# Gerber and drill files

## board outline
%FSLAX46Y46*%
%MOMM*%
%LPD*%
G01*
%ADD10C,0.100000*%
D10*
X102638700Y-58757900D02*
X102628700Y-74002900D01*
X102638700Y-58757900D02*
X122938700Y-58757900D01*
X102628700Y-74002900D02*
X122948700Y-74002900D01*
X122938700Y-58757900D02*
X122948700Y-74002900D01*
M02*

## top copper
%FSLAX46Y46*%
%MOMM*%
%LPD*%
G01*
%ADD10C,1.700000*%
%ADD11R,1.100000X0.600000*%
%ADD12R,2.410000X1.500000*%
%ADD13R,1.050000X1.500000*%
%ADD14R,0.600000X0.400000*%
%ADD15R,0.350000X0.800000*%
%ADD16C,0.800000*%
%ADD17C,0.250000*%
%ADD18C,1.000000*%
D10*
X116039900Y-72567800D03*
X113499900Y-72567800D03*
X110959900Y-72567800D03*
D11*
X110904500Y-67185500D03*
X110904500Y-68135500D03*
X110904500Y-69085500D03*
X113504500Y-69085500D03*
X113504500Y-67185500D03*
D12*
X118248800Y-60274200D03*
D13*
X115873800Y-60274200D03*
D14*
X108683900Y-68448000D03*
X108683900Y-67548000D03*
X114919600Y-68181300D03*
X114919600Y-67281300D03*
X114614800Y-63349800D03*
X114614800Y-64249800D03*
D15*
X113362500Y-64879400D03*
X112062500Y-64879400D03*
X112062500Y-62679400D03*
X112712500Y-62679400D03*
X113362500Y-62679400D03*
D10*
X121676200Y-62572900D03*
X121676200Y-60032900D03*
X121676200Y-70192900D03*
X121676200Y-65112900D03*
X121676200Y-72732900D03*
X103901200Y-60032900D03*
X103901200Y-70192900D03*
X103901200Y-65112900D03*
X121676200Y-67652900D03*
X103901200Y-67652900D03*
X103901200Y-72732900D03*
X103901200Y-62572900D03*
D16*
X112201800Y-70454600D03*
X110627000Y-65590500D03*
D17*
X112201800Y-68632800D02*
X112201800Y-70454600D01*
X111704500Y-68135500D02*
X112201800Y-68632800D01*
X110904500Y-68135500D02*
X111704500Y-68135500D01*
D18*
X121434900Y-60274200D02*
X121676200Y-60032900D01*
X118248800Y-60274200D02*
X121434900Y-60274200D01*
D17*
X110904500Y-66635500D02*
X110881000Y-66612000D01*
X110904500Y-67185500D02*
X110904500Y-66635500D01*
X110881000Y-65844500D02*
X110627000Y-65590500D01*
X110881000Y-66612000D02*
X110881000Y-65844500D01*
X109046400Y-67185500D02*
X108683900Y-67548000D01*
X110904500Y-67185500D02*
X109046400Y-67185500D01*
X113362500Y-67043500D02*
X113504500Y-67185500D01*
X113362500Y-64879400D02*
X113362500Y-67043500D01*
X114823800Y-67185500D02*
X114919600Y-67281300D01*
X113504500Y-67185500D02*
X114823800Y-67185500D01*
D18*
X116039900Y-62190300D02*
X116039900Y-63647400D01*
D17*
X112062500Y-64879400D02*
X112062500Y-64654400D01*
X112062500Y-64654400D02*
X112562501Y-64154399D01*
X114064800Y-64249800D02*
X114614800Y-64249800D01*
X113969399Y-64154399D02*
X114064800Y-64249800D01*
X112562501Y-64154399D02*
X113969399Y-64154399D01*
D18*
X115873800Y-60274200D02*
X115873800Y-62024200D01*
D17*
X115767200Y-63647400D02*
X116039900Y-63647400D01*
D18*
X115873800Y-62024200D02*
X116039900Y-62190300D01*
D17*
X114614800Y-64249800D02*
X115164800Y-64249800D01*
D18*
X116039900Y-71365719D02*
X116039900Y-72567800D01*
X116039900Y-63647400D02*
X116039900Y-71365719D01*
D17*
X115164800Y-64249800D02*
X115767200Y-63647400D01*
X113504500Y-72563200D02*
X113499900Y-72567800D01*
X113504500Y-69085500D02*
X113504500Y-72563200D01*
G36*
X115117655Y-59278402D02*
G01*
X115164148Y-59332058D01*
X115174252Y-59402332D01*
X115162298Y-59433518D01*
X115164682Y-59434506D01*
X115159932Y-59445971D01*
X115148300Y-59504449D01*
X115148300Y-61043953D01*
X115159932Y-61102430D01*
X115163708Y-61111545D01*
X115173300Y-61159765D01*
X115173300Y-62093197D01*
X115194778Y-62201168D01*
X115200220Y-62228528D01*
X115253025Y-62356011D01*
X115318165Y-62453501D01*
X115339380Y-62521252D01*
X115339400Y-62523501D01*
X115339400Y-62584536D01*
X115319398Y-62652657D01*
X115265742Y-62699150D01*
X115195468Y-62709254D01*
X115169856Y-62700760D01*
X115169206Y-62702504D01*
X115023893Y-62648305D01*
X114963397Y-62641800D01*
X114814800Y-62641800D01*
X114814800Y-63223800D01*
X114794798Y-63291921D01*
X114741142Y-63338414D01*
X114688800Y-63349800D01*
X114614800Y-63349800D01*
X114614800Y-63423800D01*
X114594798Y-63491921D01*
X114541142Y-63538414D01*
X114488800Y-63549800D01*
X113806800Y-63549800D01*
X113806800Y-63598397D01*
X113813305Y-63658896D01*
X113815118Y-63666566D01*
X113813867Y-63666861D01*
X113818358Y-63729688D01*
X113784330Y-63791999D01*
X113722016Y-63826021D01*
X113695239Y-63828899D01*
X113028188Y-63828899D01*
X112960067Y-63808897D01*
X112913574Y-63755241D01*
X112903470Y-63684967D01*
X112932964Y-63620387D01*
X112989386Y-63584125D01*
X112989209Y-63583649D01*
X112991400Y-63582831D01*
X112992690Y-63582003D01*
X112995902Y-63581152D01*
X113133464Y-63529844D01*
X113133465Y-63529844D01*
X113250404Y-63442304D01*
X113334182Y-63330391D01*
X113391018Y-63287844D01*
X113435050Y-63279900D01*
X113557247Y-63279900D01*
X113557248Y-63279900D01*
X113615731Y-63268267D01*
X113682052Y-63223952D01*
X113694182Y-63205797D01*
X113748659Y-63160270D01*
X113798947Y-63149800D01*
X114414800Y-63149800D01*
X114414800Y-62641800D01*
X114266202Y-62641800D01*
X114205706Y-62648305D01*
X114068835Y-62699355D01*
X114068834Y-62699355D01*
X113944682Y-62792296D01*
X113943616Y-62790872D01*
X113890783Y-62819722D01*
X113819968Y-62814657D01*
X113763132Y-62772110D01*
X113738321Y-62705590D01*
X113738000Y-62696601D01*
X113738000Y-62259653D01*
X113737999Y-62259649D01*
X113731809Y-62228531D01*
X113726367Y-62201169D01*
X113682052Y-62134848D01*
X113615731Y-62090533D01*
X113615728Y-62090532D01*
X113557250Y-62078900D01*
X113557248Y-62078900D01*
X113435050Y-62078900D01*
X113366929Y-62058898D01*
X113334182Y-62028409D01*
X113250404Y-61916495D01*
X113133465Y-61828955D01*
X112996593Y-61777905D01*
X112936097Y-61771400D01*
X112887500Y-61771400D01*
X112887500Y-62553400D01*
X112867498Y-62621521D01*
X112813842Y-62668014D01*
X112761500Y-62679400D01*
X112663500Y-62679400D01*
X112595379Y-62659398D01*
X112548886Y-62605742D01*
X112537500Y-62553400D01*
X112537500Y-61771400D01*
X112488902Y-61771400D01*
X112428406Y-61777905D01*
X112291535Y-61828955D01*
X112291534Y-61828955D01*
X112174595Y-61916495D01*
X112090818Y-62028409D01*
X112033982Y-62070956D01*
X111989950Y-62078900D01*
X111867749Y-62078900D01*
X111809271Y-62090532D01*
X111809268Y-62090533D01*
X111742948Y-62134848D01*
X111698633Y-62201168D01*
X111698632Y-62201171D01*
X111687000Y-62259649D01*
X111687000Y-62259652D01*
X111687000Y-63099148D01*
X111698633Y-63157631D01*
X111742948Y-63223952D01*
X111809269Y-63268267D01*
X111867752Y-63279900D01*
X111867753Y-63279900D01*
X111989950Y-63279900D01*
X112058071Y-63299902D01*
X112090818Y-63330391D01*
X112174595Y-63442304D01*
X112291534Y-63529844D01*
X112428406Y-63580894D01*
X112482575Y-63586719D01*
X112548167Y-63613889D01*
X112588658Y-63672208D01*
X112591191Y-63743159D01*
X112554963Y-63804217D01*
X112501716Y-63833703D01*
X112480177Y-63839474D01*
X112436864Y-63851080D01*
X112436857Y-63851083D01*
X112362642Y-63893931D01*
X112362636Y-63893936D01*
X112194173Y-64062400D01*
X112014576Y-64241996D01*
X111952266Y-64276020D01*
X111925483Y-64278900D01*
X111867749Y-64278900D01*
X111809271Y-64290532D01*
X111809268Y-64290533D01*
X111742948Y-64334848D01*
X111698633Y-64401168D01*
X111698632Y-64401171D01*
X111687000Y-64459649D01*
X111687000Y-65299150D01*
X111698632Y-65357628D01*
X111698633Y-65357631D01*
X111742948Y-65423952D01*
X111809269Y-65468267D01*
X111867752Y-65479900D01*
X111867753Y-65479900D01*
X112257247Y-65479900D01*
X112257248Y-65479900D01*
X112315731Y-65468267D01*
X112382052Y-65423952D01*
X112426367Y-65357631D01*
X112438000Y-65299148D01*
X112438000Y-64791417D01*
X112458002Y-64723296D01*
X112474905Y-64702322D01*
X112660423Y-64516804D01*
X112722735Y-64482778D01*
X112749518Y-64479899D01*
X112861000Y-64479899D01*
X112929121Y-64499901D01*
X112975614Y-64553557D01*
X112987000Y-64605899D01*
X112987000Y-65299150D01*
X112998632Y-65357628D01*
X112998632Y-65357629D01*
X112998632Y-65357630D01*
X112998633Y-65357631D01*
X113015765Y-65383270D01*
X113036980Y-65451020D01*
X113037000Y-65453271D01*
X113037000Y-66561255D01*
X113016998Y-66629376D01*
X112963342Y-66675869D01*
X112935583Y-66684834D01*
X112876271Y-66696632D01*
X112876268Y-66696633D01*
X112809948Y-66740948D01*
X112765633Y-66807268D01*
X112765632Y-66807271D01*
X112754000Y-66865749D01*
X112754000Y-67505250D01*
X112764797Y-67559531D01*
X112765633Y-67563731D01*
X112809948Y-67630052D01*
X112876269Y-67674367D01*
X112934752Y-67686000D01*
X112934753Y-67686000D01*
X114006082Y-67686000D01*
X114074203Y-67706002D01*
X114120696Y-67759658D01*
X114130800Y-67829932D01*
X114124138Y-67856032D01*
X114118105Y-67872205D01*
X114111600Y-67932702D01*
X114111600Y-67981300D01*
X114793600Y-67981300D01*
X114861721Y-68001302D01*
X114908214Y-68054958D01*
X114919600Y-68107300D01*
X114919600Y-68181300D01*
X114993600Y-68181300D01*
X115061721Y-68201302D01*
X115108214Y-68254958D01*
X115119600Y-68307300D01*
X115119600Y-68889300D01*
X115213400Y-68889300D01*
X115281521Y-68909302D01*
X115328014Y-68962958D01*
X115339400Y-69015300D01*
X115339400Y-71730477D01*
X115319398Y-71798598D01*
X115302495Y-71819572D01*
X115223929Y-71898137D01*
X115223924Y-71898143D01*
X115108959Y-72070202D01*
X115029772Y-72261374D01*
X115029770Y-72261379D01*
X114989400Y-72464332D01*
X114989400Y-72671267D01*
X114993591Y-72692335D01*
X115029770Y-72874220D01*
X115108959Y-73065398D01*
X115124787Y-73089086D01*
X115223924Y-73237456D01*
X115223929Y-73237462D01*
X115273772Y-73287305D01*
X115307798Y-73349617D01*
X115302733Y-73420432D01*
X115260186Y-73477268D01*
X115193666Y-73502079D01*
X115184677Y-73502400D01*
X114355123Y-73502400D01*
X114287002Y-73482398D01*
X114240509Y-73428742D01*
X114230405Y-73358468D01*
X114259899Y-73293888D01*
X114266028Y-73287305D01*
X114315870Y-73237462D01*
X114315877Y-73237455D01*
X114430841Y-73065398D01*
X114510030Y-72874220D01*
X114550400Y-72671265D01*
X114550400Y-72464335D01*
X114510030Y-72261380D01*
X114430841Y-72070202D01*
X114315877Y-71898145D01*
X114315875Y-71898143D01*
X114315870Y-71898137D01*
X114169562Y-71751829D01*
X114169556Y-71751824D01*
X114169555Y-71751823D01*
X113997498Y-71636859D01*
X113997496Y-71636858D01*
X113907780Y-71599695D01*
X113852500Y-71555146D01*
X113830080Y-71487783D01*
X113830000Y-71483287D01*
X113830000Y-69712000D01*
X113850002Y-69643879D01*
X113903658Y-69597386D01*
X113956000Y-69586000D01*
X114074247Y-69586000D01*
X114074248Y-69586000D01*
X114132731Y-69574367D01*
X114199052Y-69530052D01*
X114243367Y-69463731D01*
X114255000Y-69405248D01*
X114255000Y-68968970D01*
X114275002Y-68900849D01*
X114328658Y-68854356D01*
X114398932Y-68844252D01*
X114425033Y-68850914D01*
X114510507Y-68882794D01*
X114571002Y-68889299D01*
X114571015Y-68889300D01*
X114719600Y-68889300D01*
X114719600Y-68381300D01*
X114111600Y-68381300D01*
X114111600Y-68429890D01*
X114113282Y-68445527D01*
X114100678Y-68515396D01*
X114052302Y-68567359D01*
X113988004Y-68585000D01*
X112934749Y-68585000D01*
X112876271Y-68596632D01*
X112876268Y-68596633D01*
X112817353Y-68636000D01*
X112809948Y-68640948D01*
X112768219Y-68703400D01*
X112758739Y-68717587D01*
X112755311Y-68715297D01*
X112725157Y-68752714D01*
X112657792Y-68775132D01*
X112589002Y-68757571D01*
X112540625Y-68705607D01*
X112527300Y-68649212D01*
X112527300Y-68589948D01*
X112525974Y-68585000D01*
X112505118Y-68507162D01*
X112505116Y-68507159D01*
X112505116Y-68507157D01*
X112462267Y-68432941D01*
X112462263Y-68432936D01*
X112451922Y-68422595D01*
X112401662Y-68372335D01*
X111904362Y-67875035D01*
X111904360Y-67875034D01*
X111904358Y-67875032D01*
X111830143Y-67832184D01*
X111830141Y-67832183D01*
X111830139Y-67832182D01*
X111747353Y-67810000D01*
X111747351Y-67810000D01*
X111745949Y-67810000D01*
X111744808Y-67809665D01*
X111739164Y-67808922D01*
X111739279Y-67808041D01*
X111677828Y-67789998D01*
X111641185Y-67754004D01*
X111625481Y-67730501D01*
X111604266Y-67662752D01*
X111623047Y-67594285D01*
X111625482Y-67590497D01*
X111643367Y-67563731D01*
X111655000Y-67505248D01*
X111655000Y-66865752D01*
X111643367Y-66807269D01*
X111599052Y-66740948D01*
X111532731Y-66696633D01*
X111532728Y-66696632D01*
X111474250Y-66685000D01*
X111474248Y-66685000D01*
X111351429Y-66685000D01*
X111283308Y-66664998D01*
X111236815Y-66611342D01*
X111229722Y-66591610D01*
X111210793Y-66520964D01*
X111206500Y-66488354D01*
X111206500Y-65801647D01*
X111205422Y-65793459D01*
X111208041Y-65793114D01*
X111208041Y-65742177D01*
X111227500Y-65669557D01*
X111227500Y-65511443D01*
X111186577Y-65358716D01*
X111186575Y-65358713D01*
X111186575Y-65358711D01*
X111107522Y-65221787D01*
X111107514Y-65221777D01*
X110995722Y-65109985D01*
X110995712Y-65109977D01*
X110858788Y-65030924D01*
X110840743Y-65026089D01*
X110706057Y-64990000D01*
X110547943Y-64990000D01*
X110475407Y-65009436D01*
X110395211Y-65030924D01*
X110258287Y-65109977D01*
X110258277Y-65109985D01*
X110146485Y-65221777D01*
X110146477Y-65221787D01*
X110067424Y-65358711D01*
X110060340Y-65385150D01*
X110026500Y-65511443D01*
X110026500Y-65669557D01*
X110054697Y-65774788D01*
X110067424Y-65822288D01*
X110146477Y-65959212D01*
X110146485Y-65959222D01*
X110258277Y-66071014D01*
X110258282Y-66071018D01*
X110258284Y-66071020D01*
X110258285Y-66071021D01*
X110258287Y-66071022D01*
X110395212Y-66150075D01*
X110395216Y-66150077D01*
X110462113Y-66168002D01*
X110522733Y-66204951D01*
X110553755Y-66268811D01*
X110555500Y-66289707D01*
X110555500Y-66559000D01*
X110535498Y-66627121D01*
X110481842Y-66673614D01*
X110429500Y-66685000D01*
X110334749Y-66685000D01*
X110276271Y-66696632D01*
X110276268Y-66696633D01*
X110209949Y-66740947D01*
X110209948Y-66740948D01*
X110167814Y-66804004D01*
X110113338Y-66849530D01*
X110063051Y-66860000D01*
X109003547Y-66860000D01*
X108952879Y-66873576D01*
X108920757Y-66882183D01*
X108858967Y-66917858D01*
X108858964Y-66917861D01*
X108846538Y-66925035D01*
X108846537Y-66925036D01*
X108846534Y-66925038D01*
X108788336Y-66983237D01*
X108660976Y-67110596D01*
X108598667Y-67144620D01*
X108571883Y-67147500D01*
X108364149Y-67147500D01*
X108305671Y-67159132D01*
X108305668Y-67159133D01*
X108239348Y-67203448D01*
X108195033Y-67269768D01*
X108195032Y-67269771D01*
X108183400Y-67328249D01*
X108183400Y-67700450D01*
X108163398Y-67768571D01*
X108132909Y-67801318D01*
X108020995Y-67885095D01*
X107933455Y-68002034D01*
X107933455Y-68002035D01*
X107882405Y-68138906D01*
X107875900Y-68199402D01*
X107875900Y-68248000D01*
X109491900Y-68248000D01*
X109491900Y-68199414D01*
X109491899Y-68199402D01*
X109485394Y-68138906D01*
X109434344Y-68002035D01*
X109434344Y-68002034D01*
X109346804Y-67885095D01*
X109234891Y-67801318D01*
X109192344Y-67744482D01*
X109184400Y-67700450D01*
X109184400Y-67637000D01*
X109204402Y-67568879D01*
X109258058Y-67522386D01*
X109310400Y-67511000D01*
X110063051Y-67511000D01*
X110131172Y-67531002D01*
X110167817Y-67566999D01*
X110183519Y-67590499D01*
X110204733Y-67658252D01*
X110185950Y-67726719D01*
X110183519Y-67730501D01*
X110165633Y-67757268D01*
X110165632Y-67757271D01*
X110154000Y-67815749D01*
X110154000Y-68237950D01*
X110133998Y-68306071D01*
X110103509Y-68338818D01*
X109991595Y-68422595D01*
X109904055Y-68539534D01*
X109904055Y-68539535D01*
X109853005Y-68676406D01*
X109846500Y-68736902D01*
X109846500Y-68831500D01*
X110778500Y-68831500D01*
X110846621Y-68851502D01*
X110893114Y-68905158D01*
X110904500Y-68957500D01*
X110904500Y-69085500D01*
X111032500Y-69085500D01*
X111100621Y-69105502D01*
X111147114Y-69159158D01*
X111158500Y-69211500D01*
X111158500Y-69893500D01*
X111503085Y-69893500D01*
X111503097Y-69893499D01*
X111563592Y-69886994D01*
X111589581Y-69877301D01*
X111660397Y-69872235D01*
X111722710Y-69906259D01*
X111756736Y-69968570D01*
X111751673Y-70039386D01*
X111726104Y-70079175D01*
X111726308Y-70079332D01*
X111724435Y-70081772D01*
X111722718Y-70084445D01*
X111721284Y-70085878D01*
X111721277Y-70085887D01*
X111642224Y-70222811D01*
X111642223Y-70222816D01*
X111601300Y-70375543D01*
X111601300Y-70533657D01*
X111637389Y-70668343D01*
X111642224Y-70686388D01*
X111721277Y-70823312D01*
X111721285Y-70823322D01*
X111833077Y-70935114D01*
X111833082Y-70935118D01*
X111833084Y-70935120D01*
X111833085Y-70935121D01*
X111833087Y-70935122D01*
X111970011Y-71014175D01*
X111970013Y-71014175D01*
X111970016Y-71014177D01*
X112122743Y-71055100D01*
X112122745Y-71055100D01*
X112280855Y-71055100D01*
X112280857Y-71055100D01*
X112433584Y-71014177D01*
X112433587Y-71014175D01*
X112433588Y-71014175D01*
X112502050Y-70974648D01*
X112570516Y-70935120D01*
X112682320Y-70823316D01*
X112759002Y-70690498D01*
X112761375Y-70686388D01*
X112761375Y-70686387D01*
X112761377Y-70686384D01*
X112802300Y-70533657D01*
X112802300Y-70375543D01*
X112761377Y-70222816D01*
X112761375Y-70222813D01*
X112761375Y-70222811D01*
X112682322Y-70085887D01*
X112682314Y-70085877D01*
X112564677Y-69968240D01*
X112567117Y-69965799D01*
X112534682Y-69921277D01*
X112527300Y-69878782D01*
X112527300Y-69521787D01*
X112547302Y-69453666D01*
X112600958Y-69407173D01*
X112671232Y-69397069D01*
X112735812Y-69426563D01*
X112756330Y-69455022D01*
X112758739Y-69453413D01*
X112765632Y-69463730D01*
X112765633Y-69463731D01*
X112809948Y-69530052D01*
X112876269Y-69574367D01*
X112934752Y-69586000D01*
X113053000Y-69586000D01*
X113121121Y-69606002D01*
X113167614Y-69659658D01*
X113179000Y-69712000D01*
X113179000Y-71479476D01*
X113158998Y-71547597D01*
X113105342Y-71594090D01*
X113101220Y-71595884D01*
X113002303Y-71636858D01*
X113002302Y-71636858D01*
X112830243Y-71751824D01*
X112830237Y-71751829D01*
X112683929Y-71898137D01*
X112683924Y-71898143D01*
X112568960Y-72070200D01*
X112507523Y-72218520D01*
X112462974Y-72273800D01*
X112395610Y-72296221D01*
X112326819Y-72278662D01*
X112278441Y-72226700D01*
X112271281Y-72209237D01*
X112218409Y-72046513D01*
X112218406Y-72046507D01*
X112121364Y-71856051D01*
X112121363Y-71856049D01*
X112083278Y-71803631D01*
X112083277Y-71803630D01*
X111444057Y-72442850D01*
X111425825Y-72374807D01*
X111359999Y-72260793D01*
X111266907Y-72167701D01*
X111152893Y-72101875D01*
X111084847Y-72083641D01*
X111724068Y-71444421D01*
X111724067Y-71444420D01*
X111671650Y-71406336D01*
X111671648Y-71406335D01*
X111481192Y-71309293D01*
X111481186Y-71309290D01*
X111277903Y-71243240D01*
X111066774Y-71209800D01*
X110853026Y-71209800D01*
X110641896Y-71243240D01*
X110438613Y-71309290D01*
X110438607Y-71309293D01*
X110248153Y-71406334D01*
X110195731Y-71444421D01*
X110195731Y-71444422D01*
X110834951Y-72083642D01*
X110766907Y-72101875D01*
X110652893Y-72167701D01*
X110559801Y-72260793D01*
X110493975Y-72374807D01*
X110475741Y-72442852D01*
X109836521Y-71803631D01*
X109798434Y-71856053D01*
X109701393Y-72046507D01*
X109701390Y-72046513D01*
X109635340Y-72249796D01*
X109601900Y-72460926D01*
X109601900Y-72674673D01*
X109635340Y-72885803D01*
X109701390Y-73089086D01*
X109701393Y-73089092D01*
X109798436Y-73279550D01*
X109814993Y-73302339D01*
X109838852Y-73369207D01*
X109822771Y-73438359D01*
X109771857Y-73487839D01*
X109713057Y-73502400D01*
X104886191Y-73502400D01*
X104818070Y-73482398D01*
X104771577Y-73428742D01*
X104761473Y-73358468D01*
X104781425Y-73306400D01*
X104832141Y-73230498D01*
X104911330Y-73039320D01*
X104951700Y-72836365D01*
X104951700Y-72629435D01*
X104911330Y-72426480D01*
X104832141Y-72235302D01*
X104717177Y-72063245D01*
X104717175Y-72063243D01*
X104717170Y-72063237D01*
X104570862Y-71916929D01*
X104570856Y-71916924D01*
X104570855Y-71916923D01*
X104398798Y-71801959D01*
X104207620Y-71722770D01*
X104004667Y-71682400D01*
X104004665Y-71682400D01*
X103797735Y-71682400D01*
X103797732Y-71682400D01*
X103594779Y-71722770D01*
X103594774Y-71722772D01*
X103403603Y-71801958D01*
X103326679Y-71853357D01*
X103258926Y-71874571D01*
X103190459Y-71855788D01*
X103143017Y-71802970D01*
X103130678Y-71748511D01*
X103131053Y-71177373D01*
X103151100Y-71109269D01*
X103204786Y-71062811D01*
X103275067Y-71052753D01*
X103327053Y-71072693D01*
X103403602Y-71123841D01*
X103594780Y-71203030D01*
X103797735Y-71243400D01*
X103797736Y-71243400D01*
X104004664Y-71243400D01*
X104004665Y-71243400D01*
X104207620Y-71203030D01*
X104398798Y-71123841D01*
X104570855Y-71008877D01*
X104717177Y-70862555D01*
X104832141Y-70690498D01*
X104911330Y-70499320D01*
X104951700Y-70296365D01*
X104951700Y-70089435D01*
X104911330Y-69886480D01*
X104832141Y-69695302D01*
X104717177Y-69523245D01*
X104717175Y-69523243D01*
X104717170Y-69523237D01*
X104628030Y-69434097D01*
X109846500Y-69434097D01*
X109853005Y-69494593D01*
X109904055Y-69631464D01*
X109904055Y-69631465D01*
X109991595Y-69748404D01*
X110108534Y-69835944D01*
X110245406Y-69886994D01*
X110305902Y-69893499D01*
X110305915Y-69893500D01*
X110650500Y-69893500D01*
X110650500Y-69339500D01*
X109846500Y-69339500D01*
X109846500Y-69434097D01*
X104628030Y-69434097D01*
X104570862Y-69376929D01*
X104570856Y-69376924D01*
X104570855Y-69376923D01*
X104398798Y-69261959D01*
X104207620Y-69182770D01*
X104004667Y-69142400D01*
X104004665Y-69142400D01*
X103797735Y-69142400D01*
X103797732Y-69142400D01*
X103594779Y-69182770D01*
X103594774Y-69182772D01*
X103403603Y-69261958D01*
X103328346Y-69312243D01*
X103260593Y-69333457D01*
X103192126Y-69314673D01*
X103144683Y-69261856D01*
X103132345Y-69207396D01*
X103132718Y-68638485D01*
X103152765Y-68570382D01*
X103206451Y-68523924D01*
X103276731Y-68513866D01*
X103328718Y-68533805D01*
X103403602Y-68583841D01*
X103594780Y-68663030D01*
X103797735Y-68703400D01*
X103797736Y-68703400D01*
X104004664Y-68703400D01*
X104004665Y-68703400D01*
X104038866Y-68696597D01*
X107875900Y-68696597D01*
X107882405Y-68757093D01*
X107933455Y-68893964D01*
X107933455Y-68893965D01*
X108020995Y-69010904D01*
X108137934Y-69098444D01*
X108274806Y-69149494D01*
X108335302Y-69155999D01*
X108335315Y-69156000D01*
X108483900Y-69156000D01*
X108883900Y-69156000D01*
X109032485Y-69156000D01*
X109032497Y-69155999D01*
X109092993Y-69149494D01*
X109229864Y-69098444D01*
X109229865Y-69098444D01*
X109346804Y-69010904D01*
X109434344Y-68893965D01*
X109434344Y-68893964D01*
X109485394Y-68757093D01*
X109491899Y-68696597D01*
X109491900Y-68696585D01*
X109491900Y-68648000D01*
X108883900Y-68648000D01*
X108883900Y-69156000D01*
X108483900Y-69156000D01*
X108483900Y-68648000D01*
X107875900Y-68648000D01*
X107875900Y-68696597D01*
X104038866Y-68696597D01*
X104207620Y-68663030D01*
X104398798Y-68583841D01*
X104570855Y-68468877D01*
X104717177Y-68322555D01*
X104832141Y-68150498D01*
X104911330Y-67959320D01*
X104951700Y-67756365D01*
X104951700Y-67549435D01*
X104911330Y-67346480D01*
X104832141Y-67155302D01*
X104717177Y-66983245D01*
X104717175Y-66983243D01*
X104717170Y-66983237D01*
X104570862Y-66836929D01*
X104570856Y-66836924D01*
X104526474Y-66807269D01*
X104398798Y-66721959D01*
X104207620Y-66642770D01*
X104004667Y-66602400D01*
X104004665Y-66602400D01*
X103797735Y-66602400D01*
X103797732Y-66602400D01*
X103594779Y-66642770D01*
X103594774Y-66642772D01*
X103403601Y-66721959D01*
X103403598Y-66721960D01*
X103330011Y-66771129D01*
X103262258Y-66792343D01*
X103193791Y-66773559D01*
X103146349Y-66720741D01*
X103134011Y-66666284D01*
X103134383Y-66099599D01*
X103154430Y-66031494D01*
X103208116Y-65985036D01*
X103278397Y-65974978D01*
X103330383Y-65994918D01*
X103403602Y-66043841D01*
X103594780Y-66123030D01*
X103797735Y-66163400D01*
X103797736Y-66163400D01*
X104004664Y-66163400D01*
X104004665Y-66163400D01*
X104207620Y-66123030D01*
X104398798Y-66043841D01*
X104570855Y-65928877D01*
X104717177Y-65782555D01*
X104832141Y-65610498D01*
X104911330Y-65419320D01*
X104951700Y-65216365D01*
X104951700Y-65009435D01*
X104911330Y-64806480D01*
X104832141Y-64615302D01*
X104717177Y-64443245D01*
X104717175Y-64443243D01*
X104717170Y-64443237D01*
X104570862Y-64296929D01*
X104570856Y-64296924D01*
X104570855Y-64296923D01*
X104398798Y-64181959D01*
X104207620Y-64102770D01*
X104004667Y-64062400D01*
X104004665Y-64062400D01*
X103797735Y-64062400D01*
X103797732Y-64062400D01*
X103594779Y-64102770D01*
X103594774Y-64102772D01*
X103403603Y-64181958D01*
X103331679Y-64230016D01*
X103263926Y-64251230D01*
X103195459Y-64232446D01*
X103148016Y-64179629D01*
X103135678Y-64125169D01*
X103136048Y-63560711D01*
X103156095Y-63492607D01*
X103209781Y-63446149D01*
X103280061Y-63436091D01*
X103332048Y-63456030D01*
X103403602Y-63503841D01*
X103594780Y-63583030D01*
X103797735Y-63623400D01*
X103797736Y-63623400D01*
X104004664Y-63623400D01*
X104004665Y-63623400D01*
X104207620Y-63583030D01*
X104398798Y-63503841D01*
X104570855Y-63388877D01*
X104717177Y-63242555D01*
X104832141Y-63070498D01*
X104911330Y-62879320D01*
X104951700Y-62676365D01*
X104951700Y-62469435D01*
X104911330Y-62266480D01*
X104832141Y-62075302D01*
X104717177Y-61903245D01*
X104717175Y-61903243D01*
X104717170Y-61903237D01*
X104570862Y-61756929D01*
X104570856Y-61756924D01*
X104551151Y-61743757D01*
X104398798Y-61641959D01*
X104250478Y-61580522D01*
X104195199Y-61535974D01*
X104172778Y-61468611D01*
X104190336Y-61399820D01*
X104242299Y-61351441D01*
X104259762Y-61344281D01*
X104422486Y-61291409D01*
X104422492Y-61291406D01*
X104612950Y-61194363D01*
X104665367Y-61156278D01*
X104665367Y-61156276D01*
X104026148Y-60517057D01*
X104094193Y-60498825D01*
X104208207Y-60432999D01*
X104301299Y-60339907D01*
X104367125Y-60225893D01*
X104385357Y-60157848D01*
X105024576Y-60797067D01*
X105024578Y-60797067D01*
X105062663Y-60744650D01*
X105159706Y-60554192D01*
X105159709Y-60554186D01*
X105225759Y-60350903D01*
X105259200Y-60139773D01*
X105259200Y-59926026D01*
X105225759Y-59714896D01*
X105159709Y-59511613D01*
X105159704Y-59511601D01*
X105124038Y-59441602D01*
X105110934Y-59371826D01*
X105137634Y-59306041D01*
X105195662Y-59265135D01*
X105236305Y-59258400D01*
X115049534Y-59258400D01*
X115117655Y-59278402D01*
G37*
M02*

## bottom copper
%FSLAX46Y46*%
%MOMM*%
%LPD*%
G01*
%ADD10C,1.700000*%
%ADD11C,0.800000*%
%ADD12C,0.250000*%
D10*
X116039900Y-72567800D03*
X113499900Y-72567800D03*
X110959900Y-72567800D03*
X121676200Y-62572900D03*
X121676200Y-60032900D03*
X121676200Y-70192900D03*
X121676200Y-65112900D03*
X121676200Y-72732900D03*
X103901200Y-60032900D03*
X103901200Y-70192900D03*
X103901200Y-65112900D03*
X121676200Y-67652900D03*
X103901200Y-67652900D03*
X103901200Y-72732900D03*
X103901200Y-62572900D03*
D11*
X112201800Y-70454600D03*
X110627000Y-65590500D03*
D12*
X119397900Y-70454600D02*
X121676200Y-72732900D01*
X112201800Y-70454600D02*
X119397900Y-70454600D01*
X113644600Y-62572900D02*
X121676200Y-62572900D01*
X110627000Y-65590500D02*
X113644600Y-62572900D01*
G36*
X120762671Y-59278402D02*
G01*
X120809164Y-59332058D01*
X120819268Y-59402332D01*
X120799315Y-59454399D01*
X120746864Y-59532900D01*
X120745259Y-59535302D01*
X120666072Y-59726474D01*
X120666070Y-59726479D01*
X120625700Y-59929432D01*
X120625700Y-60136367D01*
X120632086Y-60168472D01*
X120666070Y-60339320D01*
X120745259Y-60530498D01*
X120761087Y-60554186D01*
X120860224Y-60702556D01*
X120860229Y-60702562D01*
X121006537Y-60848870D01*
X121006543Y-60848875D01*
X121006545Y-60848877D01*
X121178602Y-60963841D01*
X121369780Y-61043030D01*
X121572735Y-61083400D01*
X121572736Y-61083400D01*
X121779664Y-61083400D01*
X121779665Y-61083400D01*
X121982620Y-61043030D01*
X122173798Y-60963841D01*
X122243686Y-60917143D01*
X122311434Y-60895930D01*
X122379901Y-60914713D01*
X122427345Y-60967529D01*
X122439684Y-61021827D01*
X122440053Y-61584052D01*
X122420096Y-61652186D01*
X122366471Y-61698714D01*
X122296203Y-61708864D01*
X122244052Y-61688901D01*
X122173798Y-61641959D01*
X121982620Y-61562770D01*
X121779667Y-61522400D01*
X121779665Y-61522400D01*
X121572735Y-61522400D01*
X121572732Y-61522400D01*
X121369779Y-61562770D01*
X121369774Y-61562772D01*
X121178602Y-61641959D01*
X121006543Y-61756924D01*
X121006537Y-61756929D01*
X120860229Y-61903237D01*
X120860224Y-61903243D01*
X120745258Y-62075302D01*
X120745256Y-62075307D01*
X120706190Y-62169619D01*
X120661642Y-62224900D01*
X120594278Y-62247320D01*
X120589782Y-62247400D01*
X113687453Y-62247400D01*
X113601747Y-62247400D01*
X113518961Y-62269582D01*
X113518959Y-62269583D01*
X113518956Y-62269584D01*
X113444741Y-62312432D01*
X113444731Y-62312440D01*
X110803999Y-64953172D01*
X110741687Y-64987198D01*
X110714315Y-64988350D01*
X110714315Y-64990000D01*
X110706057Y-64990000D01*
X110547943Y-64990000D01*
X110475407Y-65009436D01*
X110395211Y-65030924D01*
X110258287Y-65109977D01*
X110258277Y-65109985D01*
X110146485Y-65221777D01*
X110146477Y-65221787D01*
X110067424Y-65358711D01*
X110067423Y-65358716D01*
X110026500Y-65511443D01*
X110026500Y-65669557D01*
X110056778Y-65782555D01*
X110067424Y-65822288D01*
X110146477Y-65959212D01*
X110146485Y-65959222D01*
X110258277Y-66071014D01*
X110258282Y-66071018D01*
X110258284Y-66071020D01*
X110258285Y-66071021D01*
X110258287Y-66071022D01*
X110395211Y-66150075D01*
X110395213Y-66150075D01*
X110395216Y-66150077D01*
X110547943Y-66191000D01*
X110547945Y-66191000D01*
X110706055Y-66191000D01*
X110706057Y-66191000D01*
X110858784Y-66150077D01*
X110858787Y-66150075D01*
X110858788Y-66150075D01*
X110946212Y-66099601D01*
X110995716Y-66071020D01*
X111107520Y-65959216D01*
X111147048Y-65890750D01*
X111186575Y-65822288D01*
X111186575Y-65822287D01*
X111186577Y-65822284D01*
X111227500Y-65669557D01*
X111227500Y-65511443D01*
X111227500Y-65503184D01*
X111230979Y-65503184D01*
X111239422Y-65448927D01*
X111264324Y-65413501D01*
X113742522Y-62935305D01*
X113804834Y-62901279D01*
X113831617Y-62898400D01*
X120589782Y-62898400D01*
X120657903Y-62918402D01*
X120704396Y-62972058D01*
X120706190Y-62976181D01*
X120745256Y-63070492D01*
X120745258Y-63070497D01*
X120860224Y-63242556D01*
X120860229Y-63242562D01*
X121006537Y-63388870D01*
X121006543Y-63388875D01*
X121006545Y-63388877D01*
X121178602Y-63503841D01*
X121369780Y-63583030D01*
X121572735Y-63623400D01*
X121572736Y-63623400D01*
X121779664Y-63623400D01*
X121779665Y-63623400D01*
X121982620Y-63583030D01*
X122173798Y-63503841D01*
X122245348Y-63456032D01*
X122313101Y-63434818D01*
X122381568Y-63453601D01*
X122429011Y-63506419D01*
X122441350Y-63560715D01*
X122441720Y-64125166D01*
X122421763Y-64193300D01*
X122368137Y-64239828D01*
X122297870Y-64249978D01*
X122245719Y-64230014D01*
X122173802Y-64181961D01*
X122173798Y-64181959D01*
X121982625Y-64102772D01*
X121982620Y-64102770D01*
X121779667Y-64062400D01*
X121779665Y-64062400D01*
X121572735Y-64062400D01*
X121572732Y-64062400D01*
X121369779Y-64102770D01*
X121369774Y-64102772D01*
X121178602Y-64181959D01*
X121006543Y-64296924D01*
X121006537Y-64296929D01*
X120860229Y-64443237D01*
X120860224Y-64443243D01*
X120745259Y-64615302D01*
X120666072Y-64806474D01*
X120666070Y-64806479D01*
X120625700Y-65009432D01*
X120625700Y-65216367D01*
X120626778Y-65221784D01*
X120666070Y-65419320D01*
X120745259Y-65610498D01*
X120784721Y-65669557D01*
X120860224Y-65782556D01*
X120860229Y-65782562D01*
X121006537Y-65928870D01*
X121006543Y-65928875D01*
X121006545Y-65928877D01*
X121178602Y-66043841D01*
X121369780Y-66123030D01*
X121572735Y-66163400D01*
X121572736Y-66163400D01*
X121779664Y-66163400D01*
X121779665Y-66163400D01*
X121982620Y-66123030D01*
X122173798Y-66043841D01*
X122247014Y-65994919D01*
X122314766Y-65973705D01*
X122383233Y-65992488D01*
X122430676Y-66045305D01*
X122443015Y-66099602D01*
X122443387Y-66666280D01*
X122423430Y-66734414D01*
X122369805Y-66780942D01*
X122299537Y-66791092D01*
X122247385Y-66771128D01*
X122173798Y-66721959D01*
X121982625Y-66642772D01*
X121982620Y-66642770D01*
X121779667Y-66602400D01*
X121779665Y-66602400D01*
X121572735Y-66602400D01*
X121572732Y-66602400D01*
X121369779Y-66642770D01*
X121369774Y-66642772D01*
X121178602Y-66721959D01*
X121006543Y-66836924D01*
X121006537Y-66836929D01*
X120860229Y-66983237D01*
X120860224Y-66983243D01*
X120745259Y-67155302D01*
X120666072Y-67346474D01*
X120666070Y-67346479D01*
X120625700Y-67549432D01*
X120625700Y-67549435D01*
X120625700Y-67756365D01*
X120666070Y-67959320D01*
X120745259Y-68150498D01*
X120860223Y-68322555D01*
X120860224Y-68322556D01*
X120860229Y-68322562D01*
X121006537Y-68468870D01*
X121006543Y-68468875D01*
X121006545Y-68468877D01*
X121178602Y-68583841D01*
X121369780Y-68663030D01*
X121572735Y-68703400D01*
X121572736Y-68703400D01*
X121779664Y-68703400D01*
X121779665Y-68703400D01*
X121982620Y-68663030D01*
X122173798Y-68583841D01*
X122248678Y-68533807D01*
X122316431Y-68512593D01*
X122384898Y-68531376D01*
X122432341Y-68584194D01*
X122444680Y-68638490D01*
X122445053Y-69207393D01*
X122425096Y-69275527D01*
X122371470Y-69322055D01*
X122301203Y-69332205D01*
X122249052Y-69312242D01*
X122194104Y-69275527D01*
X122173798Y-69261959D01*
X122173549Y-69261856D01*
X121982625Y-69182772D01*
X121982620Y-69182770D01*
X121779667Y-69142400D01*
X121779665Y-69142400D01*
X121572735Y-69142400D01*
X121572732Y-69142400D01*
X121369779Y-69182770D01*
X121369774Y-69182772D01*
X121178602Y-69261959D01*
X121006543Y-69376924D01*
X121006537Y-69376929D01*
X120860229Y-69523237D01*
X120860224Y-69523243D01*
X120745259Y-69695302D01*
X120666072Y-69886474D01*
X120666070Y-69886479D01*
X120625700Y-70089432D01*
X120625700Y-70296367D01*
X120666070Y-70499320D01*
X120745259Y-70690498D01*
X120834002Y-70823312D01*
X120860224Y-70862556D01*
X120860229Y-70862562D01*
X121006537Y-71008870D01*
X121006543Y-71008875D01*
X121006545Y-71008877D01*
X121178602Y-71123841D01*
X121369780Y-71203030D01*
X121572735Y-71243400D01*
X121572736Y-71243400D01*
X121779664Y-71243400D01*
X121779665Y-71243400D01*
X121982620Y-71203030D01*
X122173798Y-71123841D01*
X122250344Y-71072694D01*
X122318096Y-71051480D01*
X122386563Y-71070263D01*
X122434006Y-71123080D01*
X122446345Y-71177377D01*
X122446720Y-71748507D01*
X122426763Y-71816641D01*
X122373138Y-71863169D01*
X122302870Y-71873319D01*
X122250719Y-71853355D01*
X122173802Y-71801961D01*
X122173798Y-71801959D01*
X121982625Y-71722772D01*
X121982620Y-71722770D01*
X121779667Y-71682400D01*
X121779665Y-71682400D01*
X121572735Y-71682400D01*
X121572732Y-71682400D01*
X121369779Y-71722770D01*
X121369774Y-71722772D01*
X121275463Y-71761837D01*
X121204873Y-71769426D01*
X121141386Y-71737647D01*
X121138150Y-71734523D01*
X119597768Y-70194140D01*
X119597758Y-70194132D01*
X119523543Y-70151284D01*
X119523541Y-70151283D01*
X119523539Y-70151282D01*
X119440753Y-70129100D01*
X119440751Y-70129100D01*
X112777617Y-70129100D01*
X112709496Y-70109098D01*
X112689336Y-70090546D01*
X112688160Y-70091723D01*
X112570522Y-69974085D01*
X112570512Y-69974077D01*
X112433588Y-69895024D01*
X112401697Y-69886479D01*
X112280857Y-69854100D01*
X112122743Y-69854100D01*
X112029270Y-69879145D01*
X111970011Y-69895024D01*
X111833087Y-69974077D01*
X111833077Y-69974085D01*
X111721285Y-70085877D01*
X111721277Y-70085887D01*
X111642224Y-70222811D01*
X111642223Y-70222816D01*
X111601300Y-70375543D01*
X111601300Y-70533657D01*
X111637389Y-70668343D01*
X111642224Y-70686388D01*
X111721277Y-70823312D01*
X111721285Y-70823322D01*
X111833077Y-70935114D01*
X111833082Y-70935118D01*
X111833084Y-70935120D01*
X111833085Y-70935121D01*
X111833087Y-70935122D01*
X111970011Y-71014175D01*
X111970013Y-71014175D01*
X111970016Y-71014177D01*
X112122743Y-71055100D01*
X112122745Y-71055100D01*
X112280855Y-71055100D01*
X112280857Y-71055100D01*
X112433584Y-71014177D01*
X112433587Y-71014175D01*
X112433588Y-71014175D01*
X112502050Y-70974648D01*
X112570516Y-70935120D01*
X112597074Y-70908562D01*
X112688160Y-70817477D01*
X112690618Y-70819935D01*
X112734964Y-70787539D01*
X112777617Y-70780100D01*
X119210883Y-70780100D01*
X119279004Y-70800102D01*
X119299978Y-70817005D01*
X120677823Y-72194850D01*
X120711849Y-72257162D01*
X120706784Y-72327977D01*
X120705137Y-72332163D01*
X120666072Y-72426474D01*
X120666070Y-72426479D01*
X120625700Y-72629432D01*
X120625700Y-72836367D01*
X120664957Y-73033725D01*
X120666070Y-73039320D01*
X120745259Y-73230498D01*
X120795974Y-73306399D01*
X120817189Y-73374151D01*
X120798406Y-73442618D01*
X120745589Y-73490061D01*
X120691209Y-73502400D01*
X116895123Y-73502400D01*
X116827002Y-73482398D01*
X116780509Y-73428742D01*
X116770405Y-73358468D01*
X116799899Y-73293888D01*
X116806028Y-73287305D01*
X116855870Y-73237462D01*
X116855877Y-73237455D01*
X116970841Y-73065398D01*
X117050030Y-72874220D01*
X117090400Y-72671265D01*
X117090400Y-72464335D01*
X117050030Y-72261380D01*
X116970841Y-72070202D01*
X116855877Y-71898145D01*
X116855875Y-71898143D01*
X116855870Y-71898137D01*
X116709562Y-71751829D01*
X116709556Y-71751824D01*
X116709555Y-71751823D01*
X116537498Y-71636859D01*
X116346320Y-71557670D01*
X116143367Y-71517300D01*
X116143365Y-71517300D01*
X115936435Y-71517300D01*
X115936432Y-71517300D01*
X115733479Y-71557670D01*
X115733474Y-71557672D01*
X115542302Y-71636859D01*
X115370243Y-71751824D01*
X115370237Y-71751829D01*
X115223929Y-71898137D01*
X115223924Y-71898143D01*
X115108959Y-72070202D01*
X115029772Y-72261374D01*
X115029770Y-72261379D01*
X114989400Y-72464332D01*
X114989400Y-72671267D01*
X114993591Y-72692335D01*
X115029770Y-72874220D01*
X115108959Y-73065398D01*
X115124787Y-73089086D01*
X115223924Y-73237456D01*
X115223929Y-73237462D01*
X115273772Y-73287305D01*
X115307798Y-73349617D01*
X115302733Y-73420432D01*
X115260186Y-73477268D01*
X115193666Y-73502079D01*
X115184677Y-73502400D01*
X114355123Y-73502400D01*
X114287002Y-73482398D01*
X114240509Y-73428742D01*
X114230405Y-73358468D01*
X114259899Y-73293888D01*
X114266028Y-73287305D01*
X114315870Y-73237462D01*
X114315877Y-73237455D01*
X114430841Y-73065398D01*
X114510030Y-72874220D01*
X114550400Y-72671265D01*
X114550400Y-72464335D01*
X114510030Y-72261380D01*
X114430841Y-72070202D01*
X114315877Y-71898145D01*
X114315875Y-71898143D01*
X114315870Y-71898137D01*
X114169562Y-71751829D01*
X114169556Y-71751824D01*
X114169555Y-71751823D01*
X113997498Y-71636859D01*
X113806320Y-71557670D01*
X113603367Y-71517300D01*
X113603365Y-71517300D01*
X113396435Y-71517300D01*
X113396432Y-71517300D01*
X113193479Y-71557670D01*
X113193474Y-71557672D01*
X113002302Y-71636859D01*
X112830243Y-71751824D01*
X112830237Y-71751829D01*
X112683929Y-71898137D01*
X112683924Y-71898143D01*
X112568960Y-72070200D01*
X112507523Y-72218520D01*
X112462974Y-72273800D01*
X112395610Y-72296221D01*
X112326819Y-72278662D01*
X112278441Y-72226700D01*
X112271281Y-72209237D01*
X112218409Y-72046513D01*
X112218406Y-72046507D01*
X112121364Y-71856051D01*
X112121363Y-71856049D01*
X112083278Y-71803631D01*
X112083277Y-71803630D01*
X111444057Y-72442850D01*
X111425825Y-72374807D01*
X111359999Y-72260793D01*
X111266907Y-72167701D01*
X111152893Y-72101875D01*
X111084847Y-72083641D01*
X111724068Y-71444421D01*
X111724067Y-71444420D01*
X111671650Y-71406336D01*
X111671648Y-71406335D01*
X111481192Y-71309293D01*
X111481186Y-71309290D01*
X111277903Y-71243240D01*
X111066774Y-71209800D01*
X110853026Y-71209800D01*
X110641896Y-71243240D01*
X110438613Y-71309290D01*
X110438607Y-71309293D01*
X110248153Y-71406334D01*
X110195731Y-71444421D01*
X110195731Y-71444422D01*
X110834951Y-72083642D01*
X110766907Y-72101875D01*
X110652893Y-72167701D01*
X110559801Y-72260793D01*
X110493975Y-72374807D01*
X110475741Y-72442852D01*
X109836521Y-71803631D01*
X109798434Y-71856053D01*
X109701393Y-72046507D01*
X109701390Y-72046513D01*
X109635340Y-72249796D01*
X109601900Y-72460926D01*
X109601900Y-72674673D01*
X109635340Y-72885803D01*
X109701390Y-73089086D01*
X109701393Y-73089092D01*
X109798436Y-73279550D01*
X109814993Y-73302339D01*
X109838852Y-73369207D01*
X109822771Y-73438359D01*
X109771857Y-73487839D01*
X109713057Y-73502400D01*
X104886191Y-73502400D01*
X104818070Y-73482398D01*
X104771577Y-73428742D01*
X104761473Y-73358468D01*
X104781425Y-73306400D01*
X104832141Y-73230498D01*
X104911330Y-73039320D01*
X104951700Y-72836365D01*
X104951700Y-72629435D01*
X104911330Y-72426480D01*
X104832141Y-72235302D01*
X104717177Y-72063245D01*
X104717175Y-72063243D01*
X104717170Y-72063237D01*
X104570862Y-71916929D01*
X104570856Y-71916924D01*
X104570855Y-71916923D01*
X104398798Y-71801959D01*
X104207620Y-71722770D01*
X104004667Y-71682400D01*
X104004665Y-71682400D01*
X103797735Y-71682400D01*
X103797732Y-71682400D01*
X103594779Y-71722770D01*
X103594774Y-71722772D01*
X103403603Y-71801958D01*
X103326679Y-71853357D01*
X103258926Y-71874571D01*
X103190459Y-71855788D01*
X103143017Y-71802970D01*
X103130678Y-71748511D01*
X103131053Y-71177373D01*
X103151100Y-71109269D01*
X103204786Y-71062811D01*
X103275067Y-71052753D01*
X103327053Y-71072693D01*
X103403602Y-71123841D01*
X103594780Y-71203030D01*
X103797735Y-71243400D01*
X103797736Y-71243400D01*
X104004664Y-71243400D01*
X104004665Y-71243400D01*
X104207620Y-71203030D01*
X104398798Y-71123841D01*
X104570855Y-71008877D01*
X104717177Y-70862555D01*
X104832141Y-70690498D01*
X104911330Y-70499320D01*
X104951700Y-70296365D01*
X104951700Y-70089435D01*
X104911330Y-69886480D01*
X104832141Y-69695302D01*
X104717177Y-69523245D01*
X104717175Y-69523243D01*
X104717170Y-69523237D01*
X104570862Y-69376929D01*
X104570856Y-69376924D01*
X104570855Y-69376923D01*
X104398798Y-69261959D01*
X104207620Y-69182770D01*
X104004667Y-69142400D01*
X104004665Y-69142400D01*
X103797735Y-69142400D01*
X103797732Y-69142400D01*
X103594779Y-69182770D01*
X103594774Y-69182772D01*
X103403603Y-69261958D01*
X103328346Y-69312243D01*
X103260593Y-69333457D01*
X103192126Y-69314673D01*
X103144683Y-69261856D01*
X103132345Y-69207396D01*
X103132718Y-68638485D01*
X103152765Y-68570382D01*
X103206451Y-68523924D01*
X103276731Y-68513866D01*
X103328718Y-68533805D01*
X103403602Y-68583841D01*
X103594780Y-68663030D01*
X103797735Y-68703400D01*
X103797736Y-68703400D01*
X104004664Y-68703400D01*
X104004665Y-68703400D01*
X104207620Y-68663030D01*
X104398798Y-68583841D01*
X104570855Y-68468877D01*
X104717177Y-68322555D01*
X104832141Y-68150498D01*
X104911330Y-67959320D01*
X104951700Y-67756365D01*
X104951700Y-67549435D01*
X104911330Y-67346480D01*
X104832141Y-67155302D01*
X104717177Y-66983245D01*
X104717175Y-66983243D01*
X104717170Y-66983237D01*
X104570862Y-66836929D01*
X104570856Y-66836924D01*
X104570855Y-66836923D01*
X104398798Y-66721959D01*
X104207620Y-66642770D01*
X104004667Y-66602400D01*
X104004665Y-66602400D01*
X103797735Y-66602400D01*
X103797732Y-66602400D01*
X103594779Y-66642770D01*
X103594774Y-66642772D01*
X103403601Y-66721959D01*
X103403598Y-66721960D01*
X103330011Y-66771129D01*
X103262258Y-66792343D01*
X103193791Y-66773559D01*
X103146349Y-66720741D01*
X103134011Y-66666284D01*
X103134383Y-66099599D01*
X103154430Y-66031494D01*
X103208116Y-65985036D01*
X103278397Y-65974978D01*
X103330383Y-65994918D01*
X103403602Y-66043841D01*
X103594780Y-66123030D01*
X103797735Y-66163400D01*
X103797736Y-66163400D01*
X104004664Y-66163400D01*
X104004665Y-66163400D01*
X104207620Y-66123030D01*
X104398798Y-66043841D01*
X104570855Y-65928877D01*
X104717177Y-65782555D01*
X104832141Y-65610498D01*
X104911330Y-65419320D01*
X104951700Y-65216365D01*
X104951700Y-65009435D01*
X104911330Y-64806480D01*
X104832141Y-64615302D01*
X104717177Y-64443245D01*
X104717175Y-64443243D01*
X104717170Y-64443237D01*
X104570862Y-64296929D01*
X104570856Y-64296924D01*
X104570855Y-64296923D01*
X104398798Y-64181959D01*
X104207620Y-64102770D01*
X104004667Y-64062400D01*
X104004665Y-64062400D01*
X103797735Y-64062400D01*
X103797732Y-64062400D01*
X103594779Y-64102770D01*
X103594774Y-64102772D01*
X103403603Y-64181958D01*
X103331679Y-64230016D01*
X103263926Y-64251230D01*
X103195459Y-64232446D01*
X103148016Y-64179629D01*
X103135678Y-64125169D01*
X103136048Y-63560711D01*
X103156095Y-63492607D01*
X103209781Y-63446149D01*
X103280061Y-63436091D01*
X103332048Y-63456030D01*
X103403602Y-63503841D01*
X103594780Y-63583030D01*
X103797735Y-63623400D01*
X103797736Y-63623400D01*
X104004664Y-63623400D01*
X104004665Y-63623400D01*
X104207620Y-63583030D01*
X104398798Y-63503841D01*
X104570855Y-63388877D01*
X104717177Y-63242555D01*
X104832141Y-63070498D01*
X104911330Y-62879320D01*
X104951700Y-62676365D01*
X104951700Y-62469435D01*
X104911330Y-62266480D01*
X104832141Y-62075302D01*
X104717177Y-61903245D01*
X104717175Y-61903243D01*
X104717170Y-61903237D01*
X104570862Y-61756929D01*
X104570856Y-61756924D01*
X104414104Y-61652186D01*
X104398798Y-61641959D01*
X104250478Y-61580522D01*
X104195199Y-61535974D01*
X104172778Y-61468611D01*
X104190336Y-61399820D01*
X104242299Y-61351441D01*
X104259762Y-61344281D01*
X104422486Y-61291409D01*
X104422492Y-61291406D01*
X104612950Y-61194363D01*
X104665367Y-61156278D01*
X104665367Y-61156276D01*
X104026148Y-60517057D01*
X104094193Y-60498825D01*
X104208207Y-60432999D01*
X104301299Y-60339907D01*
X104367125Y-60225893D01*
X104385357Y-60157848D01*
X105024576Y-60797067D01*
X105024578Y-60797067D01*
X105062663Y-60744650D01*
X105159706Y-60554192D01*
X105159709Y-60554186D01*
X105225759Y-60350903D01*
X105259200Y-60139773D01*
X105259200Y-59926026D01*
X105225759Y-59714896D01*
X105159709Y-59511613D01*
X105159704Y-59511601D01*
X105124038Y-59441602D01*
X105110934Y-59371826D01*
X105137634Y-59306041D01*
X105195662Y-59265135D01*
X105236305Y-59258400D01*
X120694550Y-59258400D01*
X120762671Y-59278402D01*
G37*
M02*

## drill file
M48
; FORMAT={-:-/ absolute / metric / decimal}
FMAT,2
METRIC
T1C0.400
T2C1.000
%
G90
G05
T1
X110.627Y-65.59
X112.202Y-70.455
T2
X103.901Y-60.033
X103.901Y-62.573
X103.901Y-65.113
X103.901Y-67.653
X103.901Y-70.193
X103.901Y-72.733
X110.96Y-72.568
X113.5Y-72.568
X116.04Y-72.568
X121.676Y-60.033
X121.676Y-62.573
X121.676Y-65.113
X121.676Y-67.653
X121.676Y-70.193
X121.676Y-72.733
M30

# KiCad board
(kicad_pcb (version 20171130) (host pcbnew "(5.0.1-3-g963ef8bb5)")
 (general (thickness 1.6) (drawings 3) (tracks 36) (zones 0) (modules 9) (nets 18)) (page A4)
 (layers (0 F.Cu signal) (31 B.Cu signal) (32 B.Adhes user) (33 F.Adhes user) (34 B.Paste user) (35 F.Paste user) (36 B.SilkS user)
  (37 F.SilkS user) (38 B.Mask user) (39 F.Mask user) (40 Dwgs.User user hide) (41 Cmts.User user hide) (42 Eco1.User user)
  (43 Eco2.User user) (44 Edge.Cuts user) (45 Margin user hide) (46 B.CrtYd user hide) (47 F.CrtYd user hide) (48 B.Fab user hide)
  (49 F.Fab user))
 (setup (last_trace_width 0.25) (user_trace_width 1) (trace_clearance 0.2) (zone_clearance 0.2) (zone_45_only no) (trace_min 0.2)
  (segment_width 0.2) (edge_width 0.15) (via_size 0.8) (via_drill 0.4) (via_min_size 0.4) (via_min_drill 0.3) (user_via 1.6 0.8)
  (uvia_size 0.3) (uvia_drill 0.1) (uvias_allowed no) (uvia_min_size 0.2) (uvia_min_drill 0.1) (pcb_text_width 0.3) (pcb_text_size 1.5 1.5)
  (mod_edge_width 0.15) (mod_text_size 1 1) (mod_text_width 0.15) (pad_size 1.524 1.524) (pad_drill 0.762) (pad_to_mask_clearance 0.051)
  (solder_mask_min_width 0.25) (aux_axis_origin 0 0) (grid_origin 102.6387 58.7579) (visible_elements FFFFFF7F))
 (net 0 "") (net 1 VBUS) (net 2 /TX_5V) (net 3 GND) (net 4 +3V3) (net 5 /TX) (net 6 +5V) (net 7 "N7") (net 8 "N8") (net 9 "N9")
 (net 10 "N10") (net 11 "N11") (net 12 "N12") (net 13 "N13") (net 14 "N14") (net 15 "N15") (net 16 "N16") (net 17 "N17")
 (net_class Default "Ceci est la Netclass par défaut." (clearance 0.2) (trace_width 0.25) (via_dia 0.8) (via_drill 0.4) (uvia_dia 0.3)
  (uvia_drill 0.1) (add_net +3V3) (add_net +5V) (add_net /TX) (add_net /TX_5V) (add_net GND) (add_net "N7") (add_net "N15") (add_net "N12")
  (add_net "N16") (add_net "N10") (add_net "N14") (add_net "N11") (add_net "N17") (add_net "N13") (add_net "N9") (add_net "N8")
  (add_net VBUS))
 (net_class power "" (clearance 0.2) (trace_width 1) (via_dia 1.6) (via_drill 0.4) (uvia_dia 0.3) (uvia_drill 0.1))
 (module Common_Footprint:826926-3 (layer F.Cu) (at 113.4999 72.5678)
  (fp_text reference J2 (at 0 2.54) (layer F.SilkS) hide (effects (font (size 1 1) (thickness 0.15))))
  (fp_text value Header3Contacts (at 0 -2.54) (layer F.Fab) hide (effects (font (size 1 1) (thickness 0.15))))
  (pad 3 thru_hole circle (at 2.54 0) (size 1.7 1.7) (drill 1) (layers *.Cu *.Mask) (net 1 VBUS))
  (pad 2 thru_hole circle (at 0 0) (size 1.7 1.7) (drill 1) (layers *.Cu *.Mask) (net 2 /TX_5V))
  (pad 1 thru_hole circle (at -2.54 0) (size 1.7 1.7) (drill 1) (layers *.Cu *.Mask) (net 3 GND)))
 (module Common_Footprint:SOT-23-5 (layer F.Cu) (at 112.2045 68.1355)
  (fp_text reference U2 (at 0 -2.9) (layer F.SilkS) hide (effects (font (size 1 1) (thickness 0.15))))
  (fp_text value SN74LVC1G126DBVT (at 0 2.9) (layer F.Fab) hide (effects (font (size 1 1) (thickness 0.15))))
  (pad 1 smd rect (at -1.3 -0.95) (size 1.1 0.6) (layers F.Cu F.Paste F.Mask) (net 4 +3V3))
  (pad 2 smd rect (at -1.3 0) (size 1.1 0.6) (layers F.Cu F.Paste F.Mask) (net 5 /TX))
  (pad 3 smd rect (at -1.3 0.95) (size 1.1 0.6) (layers F.Cu F.Paste F.Mask) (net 3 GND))
  (pad 4 smd rect (at 1.3 0.95) (size 1.1 0.6) (layers F.Cu F.Paste F.Mask) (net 2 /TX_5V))
  (pad 5 smd rect (at 1.3 -0.95) (size 1.1 0.6) (layers F.Cu F.Paste F.Mask) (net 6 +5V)))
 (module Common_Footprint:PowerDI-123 (layer F.Cu) (at 117.3988 60.2742)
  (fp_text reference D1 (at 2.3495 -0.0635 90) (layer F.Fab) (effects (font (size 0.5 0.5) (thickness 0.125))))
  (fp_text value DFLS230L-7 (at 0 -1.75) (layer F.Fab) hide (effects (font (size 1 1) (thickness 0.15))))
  (pad 1 smd rect (at 0.85 0) (size 2.41 1.5) (layers F.Cu F.Paste F.Mask) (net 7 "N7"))
  (pad 2 smd rect (at -1.525 0) (size 1.05 1.5) (layers F.Cu F.Paste F.Mask) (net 1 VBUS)))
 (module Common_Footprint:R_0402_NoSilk (layer F.Cu) (at 108.6839 67.998 270)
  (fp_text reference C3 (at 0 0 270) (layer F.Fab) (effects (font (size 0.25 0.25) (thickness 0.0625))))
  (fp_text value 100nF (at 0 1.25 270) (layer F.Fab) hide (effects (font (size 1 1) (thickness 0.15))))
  (pad 2 smd rect (at 0.45 0 270) (size 0.4 0.6) (layers F.Cu F.Paste F.Mask) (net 3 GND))
  (pad 1 smd rect (at -0.45 0 270) (size 0.4 0.6) (layers F.Cu F.Paste F.Mask) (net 4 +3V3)))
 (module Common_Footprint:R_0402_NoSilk (layer F.Cu) (at 114.9196 67.7313 270)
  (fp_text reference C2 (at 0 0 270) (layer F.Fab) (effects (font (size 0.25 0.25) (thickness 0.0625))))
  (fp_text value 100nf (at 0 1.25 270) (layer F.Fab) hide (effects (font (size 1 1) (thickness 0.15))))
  (pad 2 smd rect (at 0.45 0 270) (size 0.4 0.6) (layers F.Cu F.Paste F.Mask) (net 3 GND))
  (pad 1 smd rect (at -0.45 0 270) (size 0.4 0.6) (layers F.Cu F.Paste F.Mask) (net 6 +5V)))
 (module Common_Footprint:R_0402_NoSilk (layer F.Cu) (at 114.6148 63.7998 90)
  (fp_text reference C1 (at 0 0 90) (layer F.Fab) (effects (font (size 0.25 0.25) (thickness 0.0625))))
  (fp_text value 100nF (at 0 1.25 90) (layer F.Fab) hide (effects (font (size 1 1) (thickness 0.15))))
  (pad 2 smd rect (at 0.45 0 90) (size 0.4 0.6) (layers F.Cu F.Paste F.Mask) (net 3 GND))
  (pad 1 smd rect (at -0.45 0 90) (size 0.4 0.6) (layers F.Cu F.Paste F.Mask) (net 1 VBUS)))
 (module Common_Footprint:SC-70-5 (layer F.Cu) (at 112.7125 63.7794 270)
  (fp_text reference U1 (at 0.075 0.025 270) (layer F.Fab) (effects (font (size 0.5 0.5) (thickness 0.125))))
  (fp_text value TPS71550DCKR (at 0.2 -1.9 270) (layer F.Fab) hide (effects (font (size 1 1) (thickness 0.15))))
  (pad 5 smd rect (at 1.1 -0.65 270) (size 0.8 0.35) (layers F.Cu F.Paste F.Mask) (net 6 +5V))
  (pad 4 smd rect (at 1.1 0.65 270) (size 0.8 0.35) (layers F.Cu F.Paste F.Mask) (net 1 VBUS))
  (pad 3 smd rect (at -1.1 0.65 270) (size 0.8 0.35) (layers F.Cu F.Paste F.Mask) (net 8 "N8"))
  (pad 2 smd rect (at -1.1 0 270) (size 0.8 0.35) (layers F.Cu F.Paste F.Mask) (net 3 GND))
  (pad 1 smd rect (at -1.1 -0.65 270) (size 0.8 0.35) (layers F.Cu F.Paste F.Mask) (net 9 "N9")))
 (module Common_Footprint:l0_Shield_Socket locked (layer F.Cu) (at 112.7887 66.3829)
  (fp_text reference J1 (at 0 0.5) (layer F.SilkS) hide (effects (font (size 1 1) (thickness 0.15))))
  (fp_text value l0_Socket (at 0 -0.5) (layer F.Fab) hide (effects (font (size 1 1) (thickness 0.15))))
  (fp_line (start -10.15 -7.625) (end -10.16 7.62) (layer Edge.Cuts) (width 0.1))
  (fp_line (start -10.15 -7.625) (end 10.15 -7.625) (layer Edge.Cuts) (width 0.1))
  (fp_line (start -10.16 7.62) (end 10.16 7.62) (layer Edge.Cuts) (width 0.1))
  (fp_line (start 10.15 -7.625) (end 10.16 7.62) (layer Edge.Cuts) (width 0.1))
  (pad 5 thru_hole circle (at 8.8875 -3.81 270) (size 1.7 1.7) (drill 1) (layers *.Cu *.Mask) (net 4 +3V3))
  (pad 6 thru_hole circle (at 8.8875 -6.35 270) (size 1.7 1.7) (drill 1) (layers *.Cu *.Mask) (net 7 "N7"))
  (pad 2 thru_hole circle (at 8.8875 3.81 270) (size 1.7 1.7) (drill 1) (layers *.Cu *.Mask) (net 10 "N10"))
  (pad 4 thru_hole circle (at 8.8875 -1.27 270) (size 1.7 1.7) (drill 1) (layers *.Cu *.Mask) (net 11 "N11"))
  (pad 1 thru_hole circle (at 8.8875 6.35 270) (size 1.7 1.7) (drill 1) (layers *.Cu *.Mask) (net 5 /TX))
  (pad 7 thru_hole circle (at -8.8875 -6.35 270) (size 1.7 1.7) (drill 1) (layers *.Cu *.Mask) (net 3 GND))
  (pad 11 thru_hole circle (at -8.8875 3.81 270) (size 1.7 1.7) (drill 1) (layers *.Cu *.Mask) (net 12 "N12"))
  (pad 9 thru_hole circle (at -8.8875 -1.27 270) (size 1.7 1.7) (drill 1) (layers *.Cu *.Mask) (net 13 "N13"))
  (pad 3 thru_hole circle (at 8.8875 1.27 270) (size 1.7 1.7) (drill 1) (layers *.Cu *.Mask) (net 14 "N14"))
  (pad 10 thru_hole circle (at -8.8875 1.27 270) (size 1.7 1.7) (drill 1) (layers *.Cu *.Mask) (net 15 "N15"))
  (pad 12 thru_hole circle (at -8.8875 6.35 270) (size 1.7 1.7) (drill 1) (layers *.Cu *.Mask) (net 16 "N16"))
  (pad 8 thru_hole circle (at -8.8875 -3.81 270) (size 1.7 1.7) (drill 1) (layers *.Cu *.Mask) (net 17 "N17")))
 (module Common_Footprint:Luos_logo (layer F.Cu) (at 108.6204 66.3271 270)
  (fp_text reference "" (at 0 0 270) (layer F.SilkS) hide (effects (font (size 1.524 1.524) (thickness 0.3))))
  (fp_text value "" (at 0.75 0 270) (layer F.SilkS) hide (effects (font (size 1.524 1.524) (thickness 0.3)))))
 (via (at 112.2018 70.4546) (size 0.8) (drill 0.4) (layers F.Cu B.Cu) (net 5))
 (segment (start 112.2018 68.6328) (end 112.2018 70.4546) (width 0.25) (layer F.Cu) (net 5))
 (segment (start 111.7045 68.1355) (end 112.2018 68.6328) (width 0.25) (layer F.Cu) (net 5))
 (segment (start 110.9045 68.1355) (end 111.7045 68.1355) (width 0.25) (layer F.Cu) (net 5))
 (segment (start 119.3979 70.4546) (end 121.6762 72.7329) (width 0.25) (layer B.Cu) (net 5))
 (segment (start 112.2018 70.4546) (end 119.3979 70.4546) (width 0.25) (layer B.Cu) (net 5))
 (segment (start 121.4349 60.2742) (end 121.6762 60.0329) (width 1) (layer F.Cu) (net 7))
 (segment (start 118.2488 60.2742) (end 121.4349 60.2742) (width 1) (layer F.Cu) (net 7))
 (segment (start 110.9045 66.6355) (end 110.881 66.612) (width 0.25) (layer F.Cu) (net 4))
 (segment (start 110.9045 67.1855) (end 110.9045 66.6355) (width 0.25) (layer F.Cu) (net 4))
 (via (at 110.627 65.5905) (size 0.8) (drill 0.4) (layers F.Cu B.Cu) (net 4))
 (segment (start 110.881 65.8445) (end 110.627 65.5905) (width 0.25) (layer F.Cu) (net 4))
 (segment (start 110.881 66.612) (end 110.881 65.8445) (width 0.25) (layer F.Cu) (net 4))
 (segment (start 113.6446 62.5729) (end 121.6762 62.5729) (width 0.25) (layer B.Cu) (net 4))
 (segment (start 110.627 65.5905) (end 113.6446 62.5729) (width 0.25) (layer B.Cu) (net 4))
 (segment (start 109.0464 67.1855) (end 108.6839 67.548) (width 0.25) (layer F.Cu) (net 4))
 (segment (start 110.9045 67.1855) (end 109.0464 67.1855) (width 0.25) (layer F.Cu) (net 4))
 (segment (start 113.3625 67.0435) (end 113.5045 67.1855) (width 0.25) (layer F.Cu) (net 6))
 (segment (start 113.3625 64.8794) (end 113.3625 67.0435) (width 0.25) (layer F.Cu) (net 6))
 (segment (start 114.8238 67.1855) (end 114.9196 67.2813) (width 0.25) (layer F.Cu) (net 6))
 (segment (start 113.5045 67.1855) (end 114.8238 67.1855) (width 0.25) (layer F.Cu) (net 6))
 (segment (start 116.0399 62.1903) (end 116.0399 63.6474) (width 1) (layer F.Cu) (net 1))
 (segment (start 112.0625 64.8794) (end 112.0625 64.6544) (width 0.25) (layer F.Cu) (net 1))
 (segment (start 112.0625 64.6544) (end 112.562501 64.154399) (width 0.25) (layer F.Cu) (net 1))
 (segment (start 114.0648 64.2498) (end 114.6148 64.2498) (width 0.25) (layer F.Cu) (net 1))
 (segment (start 113.969399 64.154399) (end 114.0648 64.2498) (width 0.25) (layer F.Cu) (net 1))
 (segment (start 112.562501 64.154399) (end 113.969399 64.154399) (width 0.25) (layer F.Cu) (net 1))
 (segment (start 115.8738 60.2742) (end 115.8738 62.0242) (width 1) (layer F.Cu) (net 1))
 (segment (start 115.7672 63.6474) (end 116.0399 63.6474) (width 0.25) (layer F.Cu) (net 1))
 (segment (start 115.8738 62.0242) (end 116.0399 62.1903) (width 1) (layer F.Cu) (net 1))
 (segment (start 114.6148 64.2498) (end 115.1648 64.2498) (width 0.25) (layer F.Cu) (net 1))
 (segment (start 116.0399 71.365719) (end 116.0399 72.5678) (width 1) (layer F.Cu) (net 1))
 (segment (start 116.0399 63.6474) (end 116.0399 71.365719) (width 1) (layer F.Cu) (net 1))
 (segment (start 115.1648 64.2498) (end 115.7672 63.6474) (width 0.25) (layer F.Cu) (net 1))
 (segment (start 113.5045 72.5632) (end 113.4999 72.5678) (width 0.25) (layer F.Cu) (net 2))
 (segment (start 113.5045 69.0855) (end 113.5045 72.5632) (width 0.25) (layer F.Cu) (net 2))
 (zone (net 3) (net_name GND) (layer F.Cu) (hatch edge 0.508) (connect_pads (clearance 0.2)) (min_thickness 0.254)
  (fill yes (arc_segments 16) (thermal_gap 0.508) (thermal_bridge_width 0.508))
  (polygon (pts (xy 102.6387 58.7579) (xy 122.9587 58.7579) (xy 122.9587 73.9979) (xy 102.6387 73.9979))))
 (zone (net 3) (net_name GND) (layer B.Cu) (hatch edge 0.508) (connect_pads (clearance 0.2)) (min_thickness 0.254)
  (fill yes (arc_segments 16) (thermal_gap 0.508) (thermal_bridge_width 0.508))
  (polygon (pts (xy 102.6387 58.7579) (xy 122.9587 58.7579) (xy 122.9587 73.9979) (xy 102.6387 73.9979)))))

